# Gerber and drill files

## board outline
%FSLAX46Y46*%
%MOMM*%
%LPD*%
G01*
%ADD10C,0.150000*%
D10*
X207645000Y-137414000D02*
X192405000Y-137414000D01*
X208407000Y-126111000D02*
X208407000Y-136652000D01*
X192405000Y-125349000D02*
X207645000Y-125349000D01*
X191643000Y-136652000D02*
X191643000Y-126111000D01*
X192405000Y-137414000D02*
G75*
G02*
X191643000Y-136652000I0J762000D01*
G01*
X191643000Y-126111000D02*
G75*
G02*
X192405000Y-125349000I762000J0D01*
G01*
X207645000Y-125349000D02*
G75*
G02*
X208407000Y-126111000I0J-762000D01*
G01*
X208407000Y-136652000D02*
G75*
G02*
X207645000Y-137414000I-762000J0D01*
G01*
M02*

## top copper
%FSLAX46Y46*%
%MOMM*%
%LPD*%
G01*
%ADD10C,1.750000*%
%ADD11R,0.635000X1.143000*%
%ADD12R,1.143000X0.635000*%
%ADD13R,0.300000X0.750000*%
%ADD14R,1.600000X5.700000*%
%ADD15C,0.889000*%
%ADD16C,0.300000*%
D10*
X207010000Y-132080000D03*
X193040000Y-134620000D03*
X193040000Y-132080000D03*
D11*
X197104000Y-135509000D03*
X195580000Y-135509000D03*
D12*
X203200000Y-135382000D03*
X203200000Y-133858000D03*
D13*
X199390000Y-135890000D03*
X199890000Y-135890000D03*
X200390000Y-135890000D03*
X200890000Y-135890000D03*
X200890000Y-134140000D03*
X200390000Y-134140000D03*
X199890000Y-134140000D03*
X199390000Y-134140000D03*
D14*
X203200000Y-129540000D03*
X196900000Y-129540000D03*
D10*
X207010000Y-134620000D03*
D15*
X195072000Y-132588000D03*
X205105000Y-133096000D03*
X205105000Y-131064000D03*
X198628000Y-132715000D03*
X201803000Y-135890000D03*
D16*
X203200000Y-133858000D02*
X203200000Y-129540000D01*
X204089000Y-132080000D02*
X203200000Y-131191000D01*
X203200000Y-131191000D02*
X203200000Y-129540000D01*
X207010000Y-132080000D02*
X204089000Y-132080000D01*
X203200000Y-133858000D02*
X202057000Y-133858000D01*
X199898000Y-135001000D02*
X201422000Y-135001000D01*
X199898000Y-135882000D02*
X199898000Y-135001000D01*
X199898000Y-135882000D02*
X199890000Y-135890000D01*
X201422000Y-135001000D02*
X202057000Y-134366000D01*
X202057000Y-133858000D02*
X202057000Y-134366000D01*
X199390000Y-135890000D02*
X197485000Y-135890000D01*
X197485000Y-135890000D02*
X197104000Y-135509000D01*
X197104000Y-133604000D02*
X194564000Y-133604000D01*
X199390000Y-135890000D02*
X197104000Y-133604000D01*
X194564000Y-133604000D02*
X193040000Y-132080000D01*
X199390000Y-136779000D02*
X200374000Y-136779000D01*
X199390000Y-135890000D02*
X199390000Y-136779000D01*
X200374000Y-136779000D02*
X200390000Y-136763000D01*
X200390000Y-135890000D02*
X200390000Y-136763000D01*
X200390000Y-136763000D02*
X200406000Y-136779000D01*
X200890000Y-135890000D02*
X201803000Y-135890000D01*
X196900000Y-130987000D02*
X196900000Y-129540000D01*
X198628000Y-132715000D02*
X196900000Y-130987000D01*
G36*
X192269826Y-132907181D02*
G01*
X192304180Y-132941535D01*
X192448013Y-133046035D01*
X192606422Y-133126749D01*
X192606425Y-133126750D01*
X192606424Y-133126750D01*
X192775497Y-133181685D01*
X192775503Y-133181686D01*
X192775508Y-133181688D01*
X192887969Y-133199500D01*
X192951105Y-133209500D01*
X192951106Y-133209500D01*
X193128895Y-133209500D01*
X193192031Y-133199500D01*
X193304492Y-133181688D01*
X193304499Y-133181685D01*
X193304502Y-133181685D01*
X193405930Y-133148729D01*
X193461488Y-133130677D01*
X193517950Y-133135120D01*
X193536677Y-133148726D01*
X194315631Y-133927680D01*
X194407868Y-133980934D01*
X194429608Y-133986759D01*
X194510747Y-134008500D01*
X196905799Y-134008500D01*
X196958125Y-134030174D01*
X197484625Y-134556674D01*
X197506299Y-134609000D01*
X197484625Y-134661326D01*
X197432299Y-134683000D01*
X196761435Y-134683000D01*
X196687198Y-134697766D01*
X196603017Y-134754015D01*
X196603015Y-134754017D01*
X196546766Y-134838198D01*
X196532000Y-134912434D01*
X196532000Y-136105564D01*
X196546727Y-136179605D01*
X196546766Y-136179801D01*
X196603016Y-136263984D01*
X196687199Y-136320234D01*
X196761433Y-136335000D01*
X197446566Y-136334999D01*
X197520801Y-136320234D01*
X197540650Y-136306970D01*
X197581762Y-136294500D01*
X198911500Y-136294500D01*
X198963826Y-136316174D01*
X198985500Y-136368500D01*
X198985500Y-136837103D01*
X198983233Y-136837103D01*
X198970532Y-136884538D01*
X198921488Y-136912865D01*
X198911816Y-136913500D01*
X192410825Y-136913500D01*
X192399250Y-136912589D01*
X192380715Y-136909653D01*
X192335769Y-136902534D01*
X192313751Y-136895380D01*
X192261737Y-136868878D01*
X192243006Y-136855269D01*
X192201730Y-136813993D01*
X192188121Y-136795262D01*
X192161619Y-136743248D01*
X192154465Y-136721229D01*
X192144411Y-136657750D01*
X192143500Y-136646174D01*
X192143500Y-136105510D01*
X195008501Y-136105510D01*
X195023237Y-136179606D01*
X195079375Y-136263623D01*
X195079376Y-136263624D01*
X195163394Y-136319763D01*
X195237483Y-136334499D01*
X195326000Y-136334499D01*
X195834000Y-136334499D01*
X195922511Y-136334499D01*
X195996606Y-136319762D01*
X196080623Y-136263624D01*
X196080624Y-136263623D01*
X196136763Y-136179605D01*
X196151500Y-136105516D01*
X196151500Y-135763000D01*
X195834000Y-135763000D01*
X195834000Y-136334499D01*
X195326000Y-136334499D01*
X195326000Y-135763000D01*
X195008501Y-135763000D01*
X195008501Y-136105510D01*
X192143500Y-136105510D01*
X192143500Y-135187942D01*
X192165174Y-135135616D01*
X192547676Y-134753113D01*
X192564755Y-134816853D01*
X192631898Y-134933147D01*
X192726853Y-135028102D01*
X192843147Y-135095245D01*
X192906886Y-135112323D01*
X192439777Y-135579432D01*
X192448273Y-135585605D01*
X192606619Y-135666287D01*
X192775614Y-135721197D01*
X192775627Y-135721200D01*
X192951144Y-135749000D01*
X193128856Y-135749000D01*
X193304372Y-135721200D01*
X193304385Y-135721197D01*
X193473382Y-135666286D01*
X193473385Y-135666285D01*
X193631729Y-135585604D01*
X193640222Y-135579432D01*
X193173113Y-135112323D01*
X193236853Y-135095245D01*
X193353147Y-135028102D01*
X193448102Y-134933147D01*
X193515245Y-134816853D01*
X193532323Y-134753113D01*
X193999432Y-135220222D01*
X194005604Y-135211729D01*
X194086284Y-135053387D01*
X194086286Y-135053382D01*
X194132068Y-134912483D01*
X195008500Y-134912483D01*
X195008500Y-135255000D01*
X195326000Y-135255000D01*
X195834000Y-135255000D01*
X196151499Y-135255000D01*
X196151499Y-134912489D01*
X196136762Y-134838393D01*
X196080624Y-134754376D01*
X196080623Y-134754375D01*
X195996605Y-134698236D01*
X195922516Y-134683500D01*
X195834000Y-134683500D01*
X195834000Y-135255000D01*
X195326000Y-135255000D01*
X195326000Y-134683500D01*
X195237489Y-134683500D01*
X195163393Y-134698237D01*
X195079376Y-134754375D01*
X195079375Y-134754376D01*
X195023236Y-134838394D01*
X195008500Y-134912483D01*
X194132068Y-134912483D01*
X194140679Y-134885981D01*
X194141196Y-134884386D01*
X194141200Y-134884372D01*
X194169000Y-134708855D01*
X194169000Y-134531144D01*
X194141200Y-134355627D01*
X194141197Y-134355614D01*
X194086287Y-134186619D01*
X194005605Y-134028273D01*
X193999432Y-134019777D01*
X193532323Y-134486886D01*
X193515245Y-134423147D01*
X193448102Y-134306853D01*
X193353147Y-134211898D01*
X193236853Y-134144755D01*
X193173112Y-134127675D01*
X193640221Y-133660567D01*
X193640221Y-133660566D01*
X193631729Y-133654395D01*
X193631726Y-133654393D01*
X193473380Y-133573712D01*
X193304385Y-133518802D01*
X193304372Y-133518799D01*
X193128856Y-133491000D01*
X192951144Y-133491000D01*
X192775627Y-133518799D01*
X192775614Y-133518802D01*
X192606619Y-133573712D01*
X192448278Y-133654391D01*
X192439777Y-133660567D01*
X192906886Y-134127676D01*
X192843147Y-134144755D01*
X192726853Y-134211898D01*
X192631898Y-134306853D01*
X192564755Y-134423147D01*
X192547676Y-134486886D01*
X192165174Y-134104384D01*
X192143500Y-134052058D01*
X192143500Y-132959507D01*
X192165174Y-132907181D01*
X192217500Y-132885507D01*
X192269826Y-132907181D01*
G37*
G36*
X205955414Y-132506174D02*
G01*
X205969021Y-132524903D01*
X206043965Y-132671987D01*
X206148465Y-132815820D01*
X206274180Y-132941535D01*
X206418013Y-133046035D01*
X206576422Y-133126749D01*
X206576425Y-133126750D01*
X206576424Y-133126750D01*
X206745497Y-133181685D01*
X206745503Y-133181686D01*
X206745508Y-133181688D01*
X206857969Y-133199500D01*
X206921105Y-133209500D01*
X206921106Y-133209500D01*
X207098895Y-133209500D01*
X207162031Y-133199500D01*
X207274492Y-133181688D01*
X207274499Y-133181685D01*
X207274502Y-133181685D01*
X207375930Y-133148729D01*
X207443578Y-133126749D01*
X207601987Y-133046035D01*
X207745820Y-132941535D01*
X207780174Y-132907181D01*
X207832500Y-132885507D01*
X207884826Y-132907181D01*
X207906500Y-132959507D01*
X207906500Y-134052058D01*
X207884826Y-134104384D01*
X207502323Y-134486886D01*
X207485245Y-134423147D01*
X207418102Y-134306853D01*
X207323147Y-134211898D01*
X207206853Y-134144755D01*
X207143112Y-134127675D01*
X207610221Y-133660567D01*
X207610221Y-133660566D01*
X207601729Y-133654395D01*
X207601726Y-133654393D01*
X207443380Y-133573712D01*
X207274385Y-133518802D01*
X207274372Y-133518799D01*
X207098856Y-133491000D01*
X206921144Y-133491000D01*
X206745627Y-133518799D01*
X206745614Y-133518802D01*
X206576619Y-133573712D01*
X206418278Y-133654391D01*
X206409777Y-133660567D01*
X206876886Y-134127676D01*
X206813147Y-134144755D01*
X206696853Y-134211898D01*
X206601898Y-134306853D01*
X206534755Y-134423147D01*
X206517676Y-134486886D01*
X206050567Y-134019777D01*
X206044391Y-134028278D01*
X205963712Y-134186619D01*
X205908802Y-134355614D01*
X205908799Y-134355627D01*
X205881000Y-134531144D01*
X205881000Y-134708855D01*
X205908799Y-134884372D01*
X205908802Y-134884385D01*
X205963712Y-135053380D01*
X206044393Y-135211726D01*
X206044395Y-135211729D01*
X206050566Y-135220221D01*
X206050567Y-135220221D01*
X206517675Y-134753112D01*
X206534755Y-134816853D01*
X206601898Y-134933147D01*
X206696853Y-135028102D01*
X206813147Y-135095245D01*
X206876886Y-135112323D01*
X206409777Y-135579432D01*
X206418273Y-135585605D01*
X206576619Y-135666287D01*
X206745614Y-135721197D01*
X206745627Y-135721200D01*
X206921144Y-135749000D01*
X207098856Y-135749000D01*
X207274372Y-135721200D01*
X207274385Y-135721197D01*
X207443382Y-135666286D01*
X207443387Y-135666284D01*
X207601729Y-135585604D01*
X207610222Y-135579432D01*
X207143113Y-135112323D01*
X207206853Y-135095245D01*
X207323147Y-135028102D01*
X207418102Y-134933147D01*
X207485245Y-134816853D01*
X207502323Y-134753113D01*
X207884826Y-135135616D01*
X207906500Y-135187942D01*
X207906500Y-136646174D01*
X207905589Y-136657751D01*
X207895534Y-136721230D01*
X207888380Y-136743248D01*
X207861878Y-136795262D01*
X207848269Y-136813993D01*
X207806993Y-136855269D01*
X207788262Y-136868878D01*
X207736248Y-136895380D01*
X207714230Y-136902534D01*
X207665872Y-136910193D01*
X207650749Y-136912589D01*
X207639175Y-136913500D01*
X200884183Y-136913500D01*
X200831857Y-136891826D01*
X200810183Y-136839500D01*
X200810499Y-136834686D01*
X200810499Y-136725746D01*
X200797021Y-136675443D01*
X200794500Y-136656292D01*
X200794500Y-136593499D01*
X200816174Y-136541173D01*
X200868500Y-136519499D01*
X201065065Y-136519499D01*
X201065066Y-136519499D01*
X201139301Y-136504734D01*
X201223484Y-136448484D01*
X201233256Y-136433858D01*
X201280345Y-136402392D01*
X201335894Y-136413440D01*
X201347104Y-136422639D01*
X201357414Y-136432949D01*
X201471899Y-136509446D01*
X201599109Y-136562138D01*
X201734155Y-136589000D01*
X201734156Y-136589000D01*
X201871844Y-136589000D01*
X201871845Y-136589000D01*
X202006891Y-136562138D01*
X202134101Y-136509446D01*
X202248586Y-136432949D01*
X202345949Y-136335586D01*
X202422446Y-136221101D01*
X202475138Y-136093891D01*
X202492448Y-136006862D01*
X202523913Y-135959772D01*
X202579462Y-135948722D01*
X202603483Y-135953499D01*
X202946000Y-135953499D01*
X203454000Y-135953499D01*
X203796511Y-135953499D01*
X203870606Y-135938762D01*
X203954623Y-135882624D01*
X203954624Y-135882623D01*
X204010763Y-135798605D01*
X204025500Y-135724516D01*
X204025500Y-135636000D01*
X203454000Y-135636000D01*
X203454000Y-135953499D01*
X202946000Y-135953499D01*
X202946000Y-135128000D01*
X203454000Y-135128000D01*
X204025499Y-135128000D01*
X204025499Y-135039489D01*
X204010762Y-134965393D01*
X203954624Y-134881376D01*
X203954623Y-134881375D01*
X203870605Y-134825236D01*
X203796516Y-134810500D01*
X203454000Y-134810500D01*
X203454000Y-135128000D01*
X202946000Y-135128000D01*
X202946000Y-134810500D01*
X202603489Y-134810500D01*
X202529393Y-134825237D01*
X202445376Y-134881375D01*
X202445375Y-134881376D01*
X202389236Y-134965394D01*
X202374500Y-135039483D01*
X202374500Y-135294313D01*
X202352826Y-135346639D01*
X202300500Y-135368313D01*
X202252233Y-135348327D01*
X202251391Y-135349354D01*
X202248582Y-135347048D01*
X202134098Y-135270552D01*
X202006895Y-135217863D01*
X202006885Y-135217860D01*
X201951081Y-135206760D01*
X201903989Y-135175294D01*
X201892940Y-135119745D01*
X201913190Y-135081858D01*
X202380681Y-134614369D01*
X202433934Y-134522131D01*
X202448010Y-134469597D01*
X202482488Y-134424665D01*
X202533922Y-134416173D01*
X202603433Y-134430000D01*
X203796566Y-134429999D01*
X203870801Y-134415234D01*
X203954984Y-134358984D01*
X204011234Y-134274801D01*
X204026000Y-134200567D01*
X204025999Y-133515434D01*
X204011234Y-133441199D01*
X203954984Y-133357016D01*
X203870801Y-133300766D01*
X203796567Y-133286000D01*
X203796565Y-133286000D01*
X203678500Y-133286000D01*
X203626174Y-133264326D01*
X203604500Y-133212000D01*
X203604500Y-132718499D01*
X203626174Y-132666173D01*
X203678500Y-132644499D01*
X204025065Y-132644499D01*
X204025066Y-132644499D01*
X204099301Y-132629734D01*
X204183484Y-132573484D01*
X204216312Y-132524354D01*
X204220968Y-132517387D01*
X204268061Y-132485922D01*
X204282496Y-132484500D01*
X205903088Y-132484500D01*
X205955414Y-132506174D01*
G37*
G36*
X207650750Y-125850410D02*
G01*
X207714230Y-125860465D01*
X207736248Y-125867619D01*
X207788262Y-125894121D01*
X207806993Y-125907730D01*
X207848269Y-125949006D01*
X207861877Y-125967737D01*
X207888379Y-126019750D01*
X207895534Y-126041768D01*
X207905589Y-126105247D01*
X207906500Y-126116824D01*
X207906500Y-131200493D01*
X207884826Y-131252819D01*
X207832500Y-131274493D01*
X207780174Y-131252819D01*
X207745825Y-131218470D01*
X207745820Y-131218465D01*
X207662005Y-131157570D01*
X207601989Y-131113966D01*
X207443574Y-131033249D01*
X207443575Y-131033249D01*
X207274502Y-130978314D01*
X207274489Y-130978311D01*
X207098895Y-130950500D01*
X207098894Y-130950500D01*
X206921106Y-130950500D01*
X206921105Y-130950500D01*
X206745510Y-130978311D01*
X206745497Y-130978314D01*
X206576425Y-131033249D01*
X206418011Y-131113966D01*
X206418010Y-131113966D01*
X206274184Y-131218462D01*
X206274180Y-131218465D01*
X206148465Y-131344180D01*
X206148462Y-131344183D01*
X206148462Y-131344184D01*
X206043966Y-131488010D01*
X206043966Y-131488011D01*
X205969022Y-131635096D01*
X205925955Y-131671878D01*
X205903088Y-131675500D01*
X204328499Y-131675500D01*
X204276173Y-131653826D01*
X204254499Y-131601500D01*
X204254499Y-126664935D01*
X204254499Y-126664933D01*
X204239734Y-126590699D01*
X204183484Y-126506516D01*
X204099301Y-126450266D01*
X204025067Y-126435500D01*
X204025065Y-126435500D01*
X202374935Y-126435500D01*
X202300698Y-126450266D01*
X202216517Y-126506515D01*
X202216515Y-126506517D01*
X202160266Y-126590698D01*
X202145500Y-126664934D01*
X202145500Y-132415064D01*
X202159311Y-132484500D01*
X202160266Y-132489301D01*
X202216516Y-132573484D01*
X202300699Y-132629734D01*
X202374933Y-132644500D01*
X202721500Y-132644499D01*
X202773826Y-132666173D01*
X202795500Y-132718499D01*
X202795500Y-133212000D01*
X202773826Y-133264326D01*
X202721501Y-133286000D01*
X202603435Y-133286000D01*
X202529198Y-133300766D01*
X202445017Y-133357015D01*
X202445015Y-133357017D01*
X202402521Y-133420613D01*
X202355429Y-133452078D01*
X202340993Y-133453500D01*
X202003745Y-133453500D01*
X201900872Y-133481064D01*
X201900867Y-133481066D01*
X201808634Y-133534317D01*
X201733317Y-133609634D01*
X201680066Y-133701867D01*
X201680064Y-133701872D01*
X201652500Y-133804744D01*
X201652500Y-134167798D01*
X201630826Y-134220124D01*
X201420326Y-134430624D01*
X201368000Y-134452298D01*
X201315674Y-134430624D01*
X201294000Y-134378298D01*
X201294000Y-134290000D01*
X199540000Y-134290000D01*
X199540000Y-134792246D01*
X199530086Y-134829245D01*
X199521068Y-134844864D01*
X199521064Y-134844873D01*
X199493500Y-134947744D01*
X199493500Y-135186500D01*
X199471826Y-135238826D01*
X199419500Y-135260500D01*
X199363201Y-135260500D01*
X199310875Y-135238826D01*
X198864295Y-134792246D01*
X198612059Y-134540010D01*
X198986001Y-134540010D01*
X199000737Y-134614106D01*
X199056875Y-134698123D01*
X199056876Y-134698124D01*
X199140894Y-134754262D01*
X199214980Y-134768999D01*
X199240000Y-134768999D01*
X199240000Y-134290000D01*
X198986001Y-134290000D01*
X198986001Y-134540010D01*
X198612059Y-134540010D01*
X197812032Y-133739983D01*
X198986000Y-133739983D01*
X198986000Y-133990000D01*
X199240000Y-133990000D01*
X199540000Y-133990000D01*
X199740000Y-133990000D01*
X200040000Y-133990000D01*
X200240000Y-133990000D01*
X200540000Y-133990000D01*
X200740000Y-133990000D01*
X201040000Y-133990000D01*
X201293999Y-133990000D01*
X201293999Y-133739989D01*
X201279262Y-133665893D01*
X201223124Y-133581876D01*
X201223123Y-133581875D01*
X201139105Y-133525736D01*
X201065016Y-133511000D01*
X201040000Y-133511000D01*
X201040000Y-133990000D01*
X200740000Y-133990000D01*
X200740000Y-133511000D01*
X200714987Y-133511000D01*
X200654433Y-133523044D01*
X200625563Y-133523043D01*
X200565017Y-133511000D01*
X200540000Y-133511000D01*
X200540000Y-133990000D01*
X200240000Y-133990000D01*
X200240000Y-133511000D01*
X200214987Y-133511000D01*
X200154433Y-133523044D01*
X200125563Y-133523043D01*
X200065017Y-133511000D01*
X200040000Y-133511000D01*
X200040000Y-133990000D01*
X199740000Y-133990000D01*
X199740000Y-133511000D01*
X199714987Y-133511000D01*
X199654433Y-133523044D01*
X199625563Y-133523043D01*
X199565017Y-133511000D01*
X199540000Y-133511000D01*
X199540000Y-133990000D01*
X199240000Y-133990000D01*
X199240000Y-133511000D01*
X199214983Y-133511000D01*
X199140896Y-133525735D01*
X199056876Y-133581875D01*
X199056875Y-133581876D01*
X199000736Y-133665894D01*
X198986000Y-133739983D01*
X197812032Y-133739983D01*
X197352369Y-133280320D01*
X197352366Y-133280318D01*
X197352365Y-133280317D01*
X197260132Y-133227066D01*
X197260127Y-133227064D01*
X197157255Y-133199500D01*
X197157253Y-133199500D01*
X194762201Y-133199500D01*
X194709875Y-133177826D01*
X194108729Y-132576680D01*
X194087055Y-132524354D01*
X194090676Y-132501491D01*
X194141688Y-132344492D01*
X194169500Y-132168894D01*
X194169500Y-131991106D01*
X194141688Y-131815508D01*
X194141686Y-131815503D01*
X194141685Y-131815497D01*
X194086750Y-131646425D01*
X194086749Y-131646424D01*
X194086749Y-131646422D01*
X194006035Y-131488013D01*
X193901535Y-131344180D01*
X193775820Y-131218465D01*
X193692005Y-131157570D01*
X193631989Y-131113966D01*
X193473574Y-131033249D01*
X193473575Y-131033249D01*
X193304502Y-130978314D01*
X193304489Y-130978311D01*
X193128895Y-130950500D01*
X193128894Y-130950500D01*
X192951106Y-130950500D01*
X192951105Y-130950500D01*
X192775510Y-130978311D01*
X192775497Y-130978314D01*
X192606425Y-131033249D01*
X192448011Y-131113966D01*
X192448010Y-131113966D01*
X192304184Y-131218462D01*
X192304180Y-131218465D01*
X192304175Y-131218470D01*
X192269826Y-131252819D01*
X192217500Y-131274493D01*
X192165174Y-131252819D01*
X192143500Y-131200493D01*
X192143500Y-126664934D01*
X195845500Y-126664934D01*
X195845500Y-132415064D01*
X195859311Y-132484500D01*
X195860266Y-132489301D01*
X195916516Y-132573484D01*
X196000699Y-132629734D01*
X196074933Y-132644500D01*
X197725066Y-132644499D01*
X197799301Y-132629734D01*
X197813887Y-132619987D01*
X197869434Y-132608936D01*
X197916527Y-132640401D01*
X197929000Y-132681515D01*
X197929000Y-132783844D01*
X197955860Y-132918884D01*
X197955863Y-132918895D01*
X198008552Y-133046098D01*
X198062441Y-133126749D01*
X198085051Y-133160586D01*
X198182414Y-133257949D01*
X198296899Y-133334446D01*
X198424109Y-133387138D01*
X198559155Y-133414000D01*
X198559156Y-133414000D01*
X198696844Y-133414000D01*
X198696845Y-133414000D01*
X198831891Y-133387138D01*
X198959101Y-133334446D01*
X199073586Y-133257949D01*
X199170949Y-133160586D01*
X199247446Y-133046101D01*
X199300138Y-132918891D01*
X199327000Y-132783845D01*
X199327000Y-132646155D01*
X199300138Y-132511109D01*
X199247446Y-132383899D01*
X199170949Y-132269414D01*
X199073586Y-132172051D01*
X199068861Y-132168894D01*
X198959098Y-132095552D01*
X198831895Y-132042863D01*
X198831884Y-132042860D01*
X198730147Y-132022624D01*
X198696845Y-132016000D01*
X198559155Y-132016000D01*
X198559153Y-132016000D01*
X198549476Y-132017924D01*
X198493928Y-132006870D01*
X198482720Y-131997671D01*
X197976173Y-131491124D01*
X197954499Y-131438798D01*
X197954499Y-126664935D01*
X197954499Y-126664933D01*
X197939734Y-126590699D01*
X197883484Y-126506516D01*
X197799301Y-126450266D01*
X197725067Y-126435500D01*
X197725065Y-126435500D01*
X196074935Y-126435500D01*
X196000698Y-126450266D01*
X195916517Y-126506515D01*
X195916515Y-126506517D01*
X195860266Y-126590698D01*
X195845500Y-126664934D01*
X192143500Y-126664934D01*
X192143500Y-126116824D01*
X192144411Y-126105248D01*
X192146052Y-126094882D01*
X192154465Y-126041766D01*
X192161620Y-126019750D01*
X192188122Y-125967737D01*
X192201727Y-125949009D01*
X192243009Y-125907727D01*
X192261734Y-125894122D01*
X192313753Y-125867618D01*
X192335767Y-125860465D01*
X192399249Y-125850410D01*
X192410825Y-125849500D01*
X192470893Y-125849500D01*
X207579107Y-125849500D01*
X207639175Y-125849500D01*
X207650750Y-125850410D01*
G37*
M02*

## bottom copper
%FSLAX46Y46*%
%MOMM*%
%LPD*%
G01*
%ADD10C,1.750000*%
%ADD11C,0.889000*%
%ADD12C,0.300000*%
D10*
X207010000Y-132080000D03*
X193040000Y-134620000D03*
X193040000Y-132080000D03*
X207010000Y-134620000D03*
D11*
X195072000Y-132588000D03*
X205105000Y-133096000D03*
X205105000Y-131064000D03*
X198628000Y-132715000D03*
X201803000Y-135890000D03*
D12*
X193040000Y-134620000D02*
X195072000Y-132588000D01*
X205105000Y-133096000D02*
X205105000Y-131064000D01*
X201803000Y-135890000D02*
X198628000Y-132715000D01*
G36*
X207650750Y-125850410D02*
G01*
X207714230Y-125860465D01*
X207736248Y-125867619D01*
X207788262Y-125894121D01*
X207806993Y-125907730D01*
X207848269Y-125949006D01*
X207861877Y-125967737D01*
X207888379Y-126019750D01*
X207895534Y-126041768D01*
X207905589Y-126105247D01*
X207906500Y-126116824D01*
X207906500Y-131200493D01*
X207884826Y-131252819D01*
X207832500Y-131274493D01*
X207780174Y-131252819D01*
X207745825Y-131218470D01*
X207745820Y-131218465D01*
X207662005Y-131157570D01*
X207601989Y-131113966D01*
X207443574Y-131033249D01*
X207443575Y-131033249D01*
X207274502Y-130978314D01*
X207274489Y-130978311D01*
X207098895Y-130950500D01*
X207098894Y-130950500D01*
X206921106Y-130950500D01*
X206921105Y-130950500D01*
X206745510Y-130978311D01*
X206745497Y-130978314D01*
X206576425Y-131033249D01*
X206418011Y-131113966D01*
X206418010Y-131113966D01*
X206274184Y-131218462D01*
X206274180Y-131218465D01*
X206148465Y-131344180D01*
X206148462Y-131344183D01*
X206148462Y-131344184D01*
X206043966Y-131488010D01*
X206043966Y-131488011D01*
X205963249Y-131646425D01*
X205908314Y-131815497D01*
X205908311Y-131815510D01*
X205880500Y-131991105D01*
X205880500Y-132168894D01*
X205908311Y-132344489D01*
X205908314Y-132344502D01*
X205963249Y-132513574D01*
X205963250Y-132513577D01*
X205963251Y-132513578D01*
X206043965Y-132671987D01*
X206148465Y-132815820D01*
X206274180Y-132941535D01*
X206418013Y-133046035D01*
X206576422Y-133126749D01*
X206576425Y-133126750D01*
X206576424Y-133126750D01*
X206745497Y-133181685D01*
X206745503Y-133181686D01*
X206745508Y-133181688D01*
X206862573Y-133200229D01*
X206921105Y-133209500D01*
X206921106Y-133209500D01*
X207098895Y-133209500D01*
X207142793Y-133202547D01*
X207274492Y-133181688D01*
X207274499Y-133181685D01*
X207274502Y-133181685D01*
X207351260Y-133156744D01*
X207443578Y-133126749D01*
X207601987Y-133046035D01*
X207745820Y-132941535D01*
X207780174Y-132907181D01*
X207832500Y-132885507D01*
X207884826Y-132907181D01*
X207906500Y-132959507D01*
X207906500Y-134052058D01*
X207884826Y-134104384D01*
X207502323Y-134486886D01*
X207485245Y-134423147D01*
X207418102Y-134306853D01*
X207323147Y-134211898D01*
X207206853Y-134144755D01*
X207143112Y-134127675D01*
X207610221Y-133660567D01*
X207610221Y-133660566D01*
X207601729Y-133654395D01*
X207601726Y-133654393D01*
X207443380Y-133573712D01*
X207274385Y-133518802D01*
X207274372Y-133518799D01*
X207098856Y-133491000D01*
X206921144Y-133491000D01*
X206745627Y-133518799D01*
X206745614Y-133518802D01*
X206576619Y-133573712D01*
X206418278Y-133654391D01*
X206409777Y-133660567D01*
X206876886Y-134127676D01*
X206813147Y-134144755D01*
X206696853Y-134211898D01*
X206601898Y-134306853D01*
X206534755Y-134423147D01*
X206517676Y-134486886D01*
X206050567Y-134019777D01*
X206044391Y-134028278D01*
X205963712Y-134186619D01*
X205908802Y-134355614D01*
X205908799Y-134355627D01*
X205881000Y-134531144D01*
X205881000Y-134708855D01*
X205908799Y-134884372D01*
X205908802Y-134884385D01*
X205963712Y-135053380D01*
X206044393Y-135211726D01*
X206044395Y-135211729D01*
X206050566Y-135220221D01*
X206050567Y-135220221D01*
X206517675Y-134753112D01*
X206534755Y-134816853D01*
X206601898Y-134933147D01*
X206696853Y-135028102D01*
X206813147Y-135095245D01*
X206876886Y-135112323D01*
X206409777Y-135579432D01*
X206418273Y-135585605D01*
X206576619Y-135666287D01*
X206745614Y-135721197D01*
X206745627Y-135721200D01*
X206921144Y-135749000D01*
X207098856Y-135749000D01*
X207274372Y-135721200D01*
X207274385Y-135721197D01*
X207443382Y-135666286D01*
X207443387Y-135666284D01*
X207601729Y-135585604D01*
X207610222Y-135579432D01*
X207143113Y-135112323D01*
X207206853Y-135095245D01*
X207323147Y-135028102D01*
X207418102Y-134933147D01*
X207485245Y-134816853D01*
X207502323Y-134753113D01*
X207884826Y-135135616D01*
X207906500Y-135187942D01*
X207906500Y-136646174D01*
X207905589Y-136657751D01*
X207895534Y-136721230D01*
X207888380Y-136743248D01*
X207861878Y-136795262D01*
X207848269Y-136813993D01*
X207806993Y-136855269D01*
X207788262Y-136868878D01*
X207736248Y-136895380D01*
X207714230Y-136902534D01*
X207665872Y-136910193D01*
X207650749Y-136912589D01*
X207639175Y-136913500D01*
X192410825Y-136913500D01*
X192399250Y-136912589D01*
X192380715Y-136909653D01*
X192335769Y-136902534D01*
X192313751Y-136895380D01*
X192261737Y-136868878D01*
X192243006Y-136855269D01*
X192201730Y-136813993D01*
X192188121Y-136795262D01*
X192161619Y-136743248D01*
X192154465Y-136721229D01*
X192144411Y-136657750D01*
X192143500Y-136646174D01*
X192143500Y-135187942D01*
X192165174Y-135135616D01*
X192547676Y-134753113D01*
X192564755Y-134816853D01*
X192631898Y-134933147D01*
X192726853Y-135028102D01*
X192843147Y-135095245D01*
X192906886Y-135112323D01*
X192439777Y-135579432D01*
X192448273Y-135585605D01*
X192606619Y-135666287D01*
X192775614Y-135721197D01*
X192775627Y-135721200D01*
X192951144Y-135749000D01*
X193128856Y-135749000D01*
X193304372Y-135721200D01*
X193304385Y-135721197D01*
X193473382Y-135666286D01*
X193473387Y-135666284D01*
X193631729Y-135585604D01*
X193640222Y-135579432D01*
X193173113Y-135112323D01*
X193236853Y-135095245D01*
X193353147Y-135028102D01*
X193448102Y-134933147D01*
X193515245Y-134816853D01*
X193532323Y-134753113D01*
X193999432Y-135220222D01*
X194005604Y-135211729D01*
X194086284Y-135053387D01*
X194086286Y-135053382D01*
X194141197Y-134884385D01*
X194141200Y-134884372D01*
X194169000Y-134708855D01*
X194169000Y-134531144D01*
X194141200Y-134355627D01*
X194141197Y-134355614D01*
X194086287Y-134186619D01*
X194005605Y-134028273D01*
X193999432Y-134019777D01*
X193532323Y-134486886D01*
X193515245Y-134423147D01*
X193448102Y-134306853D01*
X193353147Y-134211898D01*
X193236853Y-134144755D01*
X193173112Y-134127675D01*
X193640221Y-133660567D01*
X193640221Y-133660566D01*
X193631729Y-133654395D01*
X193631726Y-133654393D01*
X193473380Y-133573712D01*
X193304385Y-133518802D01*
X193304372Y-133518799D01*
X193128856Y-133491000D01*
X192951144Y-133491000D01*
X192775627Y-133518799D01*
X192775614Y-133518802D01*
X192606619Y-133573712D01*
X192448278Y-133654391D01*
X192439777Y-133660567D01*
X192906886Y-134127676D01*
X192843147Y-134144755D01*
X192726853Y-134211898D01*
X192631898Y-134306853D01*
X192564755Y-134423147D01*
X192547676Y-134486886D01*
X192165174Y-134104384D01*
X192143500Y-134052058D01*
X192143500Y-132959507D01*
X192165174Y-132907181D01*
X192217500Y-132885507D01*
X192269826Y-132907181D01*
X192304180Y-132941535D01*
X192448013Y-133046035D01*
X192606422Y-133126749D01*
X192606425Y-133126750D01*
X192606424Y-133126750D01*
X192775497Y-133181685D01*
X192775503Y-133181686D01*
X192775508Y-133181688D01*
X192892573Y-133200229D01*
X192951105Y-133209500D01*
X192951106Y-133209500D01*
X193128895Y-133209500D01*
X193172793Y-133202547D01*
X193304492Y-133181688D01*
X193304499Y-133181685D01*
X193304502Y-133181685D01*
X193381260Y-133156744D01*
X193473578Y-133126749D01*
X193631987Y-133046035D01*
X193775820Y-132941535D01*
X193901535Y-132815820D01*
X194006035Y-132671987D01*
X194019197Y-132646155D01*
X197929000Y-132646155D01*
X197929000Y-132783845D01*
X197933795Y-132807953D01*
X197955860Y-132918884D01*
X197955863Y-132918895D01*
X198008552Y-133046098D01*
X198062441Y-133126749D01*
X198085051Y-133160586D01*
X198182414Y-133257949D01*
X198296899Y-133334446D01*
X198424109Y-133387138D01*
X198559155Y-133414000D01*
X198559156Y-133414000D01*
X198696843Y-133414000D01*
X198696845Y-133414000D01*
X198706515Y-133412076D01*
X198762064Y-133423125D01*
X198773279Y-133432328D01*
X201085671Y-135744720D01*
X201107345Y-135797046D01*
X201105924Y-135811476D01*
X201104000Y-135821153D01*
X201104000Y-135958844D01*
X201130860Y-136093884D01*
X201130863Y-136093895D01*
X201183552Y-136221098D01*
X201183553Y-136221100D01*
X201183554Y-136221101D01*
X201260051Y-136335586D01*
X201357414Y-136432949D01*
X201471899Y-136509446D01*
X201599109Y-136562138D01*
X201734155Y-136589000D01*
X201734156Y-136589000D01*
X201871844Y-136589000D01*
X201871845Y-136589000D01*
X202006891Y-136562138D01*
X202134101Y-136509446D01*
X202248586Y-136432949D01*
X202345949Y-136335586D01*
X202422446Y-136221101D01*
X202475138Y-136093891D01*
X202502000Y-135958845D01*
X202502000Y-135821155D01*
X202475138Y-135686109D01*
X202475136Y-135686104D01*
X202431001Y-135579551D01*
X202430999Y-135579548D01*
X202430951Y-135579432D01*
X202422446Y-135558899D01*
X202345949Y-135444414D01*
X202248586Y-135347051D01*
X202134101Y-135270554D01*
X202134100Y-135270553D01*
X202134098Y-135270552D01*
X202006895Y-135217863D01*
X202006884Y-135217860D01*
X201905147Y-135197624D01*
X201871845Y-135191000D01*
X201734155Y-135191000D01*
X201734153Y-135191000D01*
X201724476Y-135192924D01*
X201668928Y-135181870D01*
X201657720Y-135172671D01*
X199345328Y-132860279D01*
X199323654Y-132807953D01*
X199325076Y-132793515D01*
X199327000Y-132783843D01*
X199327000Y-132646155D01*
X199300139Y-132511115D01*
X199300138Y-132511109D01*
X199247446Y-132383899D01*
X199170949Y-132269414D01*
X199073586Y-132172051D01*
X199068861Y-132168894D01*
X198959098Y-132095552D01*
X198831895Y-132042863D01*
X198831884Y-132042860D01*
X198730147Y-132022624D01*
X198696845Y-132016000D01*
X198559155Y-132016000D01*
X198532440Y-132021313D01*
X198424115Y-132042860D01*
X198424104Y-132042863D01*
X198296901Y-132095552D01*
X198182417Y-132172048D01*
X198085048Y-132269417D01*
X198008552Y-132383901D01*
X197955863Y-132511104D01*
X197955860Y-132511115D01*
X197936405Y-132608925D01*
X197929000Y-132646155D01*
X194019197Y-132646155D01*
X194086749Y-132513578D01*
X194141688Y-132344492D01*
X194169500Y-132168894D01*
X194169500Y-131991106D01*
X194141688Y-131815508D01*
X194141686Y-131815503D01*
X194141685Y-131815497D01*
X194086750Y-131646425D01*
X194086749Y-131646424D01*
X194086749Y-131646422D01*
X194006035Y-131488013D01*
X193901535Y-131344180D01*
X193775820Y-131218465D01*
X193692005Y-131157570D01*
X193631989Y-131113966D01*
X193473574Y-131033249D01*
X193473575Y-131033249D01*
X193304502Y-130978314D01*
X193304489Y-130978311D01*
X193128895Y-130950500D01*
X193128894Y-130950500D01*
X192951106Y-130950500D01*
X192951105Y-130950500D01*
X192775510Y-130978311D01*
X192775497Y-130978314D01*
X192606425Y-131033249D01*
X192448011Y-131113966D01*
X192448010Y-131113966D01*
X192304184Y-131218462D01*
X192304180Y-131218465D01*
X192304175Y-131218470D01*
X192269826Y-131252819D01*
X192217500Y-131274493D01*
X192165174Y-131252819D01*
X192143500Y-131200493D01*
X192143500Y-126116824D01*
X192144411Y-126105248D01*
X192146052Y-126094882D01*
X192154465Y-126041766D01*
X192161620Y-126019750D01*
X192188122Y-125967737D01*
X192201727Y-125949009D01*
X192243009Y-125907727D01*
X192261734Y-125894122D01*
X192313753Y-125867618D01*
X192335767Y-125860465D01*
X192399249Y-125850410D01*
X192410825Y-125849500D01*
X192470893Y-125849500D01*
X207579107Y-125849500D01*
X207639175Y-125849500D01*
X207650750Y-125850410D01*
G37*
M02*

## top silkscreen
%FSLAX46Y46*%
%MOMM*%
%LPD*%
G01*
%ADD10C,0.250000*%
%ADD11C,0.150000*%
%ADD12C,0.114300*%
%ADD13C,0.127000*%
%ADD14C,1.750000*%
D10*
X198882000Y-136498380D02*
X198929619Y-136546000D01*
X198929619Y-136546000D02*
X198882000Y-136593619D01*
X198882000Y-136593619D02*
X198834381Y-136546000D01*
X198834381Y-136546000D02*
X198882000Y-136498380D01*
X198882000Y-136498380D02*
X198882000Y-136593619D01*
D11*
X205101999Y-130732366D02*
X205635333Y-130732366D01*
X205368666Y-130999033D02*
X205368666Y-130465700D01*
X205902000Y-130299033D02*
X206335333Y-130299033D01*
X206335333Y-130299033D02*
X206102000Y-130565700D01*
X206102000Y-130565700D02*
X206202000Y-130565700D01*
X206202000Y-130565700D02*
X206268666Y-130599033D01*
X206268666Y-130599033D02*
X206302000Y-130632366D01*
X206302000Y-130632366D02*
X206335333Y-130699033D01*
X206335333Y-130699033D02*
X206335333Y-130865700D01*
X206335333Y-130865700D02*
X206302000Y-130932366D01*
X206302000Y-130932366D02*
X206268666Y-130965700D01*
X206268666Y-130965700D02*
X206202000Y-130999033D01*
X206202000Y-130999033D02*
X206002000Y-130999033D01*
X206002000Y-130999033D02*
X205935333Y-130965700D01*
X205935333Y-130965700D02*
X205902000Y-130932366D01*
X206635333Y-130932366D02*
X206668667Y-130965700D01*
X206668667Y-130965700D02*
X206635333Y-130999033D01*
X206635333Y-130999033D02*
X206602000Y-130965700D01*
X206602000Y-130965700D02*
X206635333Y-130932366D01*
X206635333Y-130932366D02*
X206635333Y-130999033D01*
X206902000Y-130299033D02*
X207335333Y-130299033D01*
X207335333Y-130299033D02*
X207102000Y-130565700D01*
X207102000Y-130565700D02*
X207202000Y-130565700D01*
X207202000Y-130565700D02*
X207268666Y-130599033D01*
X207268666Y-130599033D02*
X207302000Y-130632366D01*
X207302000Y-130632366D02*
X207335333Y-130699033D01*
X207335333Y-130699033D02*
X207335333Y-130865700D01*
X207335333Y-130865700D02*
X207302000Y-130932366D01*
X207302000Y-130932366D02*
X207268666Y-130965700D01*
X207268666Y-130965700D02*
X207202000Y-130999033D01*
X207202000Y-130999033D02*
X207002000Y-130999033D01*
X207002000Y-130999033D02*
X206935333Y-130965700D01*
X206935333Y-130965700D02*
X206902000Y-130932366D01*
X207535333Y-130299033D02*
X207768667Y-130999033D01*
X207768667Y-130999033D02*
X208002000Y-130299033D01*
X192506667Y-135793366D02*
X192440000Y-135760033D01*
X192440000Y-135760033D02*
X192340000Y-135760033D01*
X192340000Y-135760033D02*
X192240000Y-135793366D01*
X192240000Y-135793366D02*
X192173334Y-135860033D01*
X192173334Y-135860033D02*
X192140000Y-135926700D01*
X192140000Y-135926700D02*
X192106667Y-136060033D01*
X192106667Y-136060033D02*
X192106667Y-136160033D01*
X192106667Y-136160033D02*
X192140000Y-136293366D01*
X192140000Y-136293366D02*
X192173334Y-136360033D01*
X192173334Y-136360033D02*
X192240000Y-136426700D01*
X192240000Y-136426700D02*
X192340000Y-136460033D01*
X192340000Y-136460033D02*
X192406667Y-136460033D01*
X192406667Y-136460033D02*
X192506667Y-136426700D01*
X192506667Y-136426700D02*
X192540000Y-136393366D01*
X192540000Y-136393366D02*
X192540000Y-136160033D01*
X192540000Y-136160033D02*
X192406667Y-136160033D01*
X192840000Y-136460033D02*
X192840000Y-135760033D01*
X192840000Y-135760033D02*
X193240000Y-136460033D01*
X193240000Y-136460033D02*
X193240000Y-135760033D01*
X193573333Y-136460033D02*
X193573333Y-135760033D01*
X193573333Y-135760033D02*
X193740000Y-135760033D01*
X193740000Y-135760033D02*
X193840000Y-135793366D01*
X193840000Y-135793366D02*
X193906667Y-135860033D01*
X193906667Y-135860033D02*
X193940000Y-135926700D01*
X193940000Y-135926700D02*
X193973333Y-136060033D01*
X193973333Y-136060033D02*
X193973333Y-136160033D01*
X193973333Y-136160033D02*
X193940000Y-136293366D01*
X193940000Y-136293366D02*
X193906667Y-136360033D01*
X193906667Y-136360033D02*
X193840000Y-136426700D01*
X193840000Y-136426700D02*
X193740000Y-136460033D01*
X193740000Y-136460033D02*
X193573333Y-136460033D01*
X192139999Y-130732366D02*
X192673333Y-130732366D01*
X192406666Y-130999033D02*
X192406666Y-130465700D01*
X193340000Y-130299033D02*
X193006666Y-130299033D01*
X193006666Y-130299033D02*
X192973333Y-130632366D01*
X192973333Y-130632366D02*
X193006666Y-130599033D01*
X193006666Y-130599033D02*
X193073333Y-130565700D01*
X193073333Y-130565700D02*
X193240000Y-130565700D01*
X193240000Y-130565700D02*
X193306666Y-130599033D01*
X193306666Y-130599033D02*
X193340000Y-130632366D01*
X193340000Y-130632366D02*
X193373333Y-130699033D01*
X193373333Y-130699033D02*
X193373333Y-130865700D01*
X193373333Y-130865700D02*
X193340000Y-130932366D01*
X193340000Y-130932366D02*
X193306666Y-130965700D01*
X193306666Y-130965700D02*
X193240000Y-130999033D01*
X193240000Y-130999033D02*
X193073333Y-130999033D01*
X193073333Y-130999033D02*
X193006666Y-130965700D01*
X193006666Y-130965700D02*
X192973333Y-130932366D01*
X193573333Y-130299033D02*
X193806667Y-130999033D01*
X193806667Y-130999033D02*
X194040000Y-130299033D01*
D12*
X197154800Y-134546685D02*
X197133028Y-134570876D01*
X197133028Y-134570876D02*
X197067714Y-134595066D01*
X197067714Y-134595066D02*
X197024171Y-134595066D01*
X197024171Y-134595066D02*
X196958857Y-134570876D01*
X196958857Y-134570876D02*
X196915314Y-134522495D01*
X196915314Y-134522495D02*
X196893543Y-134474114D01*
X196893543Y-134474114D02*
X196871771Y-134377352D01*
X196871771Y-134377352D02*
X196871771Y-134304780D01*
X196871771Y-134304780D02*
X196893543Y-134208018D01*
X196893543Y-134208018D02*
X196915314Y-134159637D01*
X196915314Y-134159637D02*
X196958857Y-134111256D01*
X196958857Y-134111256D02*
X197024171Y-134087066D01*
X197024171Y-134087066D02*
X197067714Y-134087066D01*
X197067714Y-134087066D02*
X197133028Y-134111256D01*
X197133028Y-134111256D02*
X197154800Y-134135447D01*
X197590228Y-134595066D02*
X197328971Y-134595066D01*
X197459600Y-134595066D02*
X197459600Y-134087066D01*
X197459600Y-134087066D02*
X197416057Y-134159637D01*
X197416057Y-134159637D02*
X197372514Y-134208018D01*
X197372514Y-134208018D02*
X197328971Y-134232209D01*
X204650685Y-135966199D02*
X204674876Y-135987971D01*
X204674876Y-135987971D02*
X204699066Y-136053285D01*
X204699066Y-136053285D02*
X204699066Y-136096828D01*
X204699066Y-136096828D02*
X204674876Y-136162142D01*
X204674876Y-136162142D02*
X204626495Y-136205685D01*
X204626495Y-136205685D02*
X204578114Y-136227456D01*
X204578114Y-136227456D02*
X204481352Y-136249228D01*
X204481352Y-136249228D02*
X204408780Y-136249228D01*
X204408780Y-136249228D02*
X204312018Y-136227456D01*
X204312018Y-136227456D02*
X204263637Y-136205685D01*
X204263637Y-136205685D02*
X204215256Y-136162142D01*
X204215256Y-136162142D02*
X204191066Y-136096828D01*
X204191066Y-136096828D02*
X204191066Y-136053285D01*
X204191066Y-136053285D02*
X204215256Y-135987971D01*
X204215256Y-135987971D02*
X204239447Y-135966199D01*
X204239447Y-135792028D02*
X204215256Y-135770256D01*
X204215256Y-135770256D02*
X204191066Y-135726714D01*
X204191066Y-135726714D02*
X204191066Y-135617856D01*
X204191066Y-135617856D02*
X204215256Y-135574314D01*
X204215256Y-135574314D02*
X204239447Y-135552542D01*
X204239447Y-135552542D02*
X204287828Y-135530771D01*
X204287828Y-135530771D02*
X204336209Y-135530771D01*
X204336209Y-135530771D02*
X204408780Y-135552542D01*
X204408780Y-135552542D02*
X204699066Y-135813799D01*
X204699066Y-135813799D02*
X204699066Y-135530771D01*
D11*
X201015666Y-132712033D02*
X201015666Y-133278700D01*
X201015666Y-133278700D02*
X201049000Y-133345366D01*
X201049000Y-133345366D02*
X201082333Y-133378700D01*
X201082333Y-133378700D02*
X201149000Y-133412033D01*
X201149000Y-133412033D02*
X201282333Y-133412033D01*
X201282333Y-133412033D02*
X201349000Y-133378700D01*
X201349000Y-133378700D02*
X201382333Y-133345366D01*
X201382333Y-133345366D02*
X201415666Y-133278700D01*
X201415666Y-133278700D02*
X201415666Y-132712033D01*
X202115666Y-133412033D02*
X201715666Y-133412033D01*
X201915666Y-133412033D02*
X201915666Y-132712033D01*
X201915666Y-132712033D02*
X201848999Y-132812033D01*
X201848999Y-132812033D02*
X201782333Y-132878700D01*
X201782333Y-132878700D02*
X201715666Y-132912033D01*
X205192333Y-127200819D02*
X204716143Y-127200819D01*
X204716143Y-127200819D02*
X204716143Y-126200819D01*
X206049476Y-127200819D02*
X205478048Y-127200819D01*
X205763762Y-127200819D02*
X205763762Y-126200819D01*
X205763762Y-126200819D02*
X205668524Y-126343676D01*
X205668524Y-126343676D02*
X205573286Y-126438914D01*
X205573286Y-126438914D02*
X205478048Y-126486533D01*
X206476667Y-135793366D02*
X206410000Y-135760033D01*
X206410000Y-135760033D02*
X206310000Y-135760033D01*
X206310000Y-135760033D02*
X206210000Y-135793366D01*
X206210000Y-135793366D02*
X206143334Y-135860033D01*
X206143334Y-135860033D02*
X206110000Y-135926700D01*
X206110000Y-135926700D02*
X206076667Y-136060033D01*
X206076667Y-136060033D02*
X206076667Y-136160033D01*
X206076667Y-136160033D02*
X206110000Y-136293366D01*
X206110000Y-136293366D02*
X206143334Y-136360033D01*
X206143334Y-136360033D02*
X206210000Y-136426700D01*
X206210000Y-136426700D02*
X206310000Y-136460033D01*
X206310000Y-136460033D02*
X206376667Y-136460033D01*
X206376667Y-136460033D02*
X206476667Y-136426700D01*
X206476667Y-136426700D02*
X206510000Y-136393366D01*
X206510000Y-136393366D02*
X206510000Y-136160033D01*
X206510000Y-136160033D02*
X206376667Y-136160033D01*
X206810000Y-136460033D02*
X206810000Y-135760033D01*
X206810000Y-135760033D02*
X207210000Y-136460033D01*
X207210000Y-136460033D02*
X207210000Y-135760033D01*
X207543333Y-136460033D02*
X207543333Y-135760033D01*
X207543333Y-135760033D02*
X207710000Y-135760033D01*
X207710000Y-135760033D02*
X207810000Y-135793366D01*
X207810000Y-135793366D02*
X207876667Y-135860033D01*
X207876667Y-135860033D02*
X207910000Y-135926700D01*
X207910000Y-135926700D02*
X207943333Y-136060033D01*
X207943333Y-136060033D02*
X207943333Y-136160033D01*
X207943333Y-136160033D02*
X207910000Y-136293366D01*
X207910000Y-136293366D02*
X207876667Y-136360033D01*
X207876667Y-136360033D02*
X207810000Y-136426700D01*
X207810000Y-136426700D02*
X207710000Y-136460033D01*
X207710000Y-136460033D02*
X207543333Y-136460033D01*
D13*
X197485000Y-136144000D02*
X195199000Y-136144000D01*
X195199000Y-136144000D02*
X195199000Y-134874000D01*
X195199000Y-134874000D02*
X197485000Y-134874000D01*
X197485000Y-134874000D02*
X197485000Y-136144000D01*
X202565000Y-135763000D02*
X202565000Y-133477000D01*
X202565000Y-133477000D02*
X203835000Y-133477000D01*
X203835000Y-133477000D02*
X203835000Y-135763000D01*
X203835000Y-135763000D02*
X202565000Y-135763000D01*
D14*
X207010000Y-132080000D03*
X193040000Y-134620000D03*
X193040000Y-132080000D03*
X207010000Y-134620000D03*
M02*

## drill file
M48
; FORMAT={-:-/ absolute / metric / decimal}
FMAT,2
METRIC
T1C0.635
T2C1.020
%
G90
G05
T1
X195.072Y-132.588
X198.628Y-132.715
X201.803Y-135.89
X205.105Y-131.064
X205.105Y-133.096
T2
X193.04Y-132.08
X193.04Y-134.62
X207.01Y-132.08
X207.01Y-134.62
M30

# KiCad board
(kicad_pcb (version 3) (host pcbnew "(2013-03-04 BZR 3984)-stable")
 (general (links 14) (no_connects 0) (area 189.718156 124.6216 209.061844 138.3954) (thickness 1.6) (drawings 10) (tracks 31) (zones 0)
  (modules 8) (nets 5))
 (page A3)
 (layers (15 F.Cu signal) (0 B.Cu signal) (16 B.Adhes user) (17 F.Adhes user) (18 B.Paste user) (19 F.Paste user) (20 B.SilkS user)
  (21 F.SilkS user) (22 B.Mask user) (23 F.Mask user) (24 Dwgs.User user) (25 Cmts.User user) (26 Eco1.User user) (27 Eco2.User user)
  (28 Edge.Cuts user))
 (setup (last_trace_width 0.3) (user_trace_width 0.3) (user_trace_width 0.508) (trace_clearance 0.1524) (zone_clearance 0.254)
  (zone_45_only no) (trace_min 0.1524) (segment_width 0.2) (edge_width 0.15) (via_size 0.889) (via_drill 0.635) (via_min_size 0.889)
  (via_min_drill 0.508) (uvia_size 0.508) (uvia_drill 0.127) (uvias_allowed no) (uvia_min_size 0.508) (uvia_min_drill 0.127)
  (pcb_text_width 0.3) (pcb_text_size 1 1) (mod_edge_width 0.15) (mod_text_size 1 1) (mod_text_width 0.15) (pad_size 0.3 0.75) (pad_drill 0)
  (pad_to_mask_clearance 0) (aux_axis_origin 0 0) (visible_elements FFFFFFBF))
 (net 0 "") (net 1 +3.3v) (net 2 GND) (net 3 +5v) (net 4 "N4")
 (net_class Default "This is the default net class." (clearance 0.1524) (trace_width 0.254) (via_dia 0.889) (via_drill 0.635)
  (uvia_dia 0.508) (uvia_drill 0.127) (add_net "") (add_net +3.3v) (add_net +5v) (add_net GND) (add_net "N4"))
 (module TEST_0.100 (layer F.Cu) (at 207.01 132.08)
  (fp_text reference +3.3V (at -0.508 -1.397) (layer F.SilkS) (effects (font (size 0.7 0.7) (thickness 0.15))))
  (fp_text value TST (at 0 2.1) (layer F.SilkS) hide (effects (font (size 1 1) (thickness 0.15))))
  (pad 1 thru_hole circle (at 0 0) (size 1.75 1.75) (drill 1.02) (layers *.Cu *.Mask F.SilkS) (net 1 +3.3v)))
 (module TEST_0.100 (layer F.Cu) (at 193.04 134.62)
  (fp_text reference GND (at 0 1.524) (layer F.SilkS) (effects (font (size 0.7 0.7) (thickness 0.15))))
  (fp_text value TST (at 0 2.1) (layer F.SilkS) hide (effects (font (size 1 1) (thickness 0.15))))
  (pad 1 thru_hole circle (at 0 0) (size 1.75 1.75) (drill 1.02) (layers *.Cu *.Mask F.SilkS) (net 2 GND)))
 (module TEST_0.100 (layer F.Cu) (at 193.04 132.08)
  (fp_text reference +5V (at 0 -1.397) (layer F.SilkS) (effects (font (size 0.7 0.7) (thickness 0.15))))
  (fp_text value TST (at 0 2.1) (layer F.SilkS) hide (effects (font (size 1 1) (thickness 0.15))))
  (pad 1 thru_hole circle (at 0 0) (size 1.75 1.75) (drill 1.02) (layers *.Cu *.Mask F.SilkS) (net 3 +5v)))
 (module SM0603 (layer F.Cu) (at 196.342 135.509 180)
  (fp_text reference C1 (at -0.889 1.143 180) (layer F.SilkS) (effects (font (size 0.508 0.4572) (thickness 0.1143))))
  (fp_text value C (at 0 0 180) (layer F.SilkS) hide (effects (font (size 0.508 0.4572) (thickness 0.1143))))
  (fp_line (start -1.143 -0.635) (end 1.143 -0.635) (layer F.SilkS) (width 0.127))
  (fp_line (start 1.143 -0.635) (end 1.143 0.635) (layer F.SilkS) (width 0.127))
  (fp_line (start 1.143 0.635) (end -1.143 0.635) (layer F.SilkS) (width 0.127))
  (fp_line (start -1.143 0.635) (end -1.143 -0.635) (layer F.SilkS) (width 0.127))
  (pad 1 smd rect (at -0.762 0 180) (size 0.635 1.143) (layers F.Cu F.Paste F.Mask) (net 3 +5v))
  (pad 2 smd rect (at 0.762 0 180) (size 0.635 1.143) (layers F.Cu F.Paste F.Mask) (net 2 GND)))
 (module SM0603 (layer F.Cu) (at 203.2 134.62 90)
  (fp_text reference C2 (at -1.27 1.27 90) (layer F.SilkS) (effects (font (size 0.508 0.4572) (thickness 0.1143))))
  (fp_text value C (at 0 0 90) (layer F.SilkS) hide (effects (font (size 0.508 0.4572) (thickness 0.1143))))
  (fp_line (start -1.143 -0.635) (end 1.143 -0.635) (layer F.SilkS) (width 0.127))
  (fp_line (start 1.143 -0.635) (end 1.143 0.635) (layer F.SilkS) (width 0.127))
  (fp_line (start 1.143 0.635) (end -1.143 0.635) (layer F.SilkS) (width 0.127))
  (fp_line (start -1.143 0.635) (end -1.143 -0.635) (layer F.SilkS) (width 0.127))
  (pad 1 smd rect (at -0.762 0 90) (size 0.635 1.143) (layers F.Cu F.Paste F.Mask) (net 2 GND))
  (pad 2 smd rect (at 0.762 0 90) (size 0.635 1.143) (layers F.Cu F.Paste F.Mask) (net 1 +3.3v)))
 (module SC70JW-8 (layer F.Cu) (at 199.39 135.89)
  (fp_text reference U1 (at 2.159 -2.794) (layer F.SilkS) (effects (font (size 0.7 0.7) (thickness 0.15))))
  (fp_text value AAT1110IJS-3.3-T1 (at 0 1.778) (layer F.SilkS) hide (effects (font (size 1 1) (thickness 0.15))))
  (pad 1 smd rect (at 0 0) (size 0.3 0.75) (layers F.Cu F.Paste F.Mask) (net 3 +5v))
  (pad 2 smd rect (at 0.5 0) (size 0.3 0.75) (layers F.Cu F.Paste F.Mask) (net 1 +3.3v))
  (pad 3 smd rect (at 1 0) (size 0.3 0.75) (layers F.Cu F.Paste F.Mask) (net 3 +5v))
  (pad 4 smd rect (at 1.5 0) (size 0.3 0.75) (layers F.Cu F.Paste F.Mask) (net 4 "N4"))
  (pad 5 smd rect (at 1.5 -1.75) (size 0.3 0.75) (layers F.Cu F.Paste F.Mask) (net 2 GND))
  (pad 6 smd rect (at 1 -1.75) (size 0.3 0.75) (layers F.Cu F.Paste F.Mask) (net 2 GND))
  (pad 7 smd rect (at 0.5 -1.75) (size 0.3 0.75) (layers F.Cu F.Paste F.Mask) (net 2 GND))
  (pad 8 smd rect (at 0 -1.75) (size 0.3 0.75) (layers F.Cu F.Paste F.Mask) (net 2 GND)))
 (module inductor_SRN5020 (layer F.Cu) (at 203.2 129.54 180)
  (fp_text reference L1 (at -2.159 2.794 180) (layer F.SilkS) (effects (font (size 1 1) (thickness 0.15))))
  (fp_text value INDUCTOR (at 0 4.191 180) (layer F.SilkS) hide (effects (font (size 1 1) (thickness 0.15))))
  (pad 1 smd rect (at 0 0 180) (size 1.6 5.7) (layers F.Cu F.Paste F.Mask) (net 1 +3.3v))
  (pad 2 smd rect (at 6.3 0 180) (size 1.6 5.7) (layers F.Cu F.Paste F.Mask) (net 4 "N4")))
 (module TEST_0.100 (layer F.Cu) (at 207.01 134.62)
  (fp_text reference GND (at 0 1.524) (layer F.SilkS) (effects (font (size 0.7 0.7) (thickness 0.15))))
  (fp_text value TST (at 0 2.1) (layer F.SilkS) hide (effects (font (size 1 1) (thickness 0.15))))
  (pad 1 thru_hole circle (at 0 0) (size 1.75 1.75) (drill 1.02) (layers *.Cu *.Mask F.SilkS) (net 2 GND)))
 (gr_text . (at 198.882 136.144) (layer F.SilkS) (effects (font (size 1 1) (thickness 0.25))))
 (gr_line (start 207.645 137.414) (end 192.405 137.414) (angle 90) (layer Edge.Cuts) (width 0.15))
 (gr_line (start 208.407 126.111) (end 208.407 136.652) (angle 90) (layer Edge.Cuts) (width 0.15))
 (gr_line (start 192.405 125.349) (end 207.645 125.349) (angle 90) (layer Edge.Cuts) (width 0.15))
 (gr_line (start 191.643 136.652) (end 191.643 126.111) (angle 90) (layer Edge.Cuts) (width 0.15))
 (gr_arc (start 192.405 136.652) (end 192.405 137.414) (angle 90) (layer Edge.Cuts) (width 0.15))
 (gr_arc (start 192.405 126.111) (end 191.643 126.111) (angle 90) (layer Edge.Cuts) (width 0.15))
 (gr_arc (start 207.645 126.111) (end 207.645 125.349) (angle 90) (layer Edge.Cuts) (width 0.15))
 (gr_arc (start 207.645 136.652) (end 208.407 136.652) (angle 90) (layer Edge.Cuts) (width 0.15))
 (segment (start 203.2 133.858) (end 203.2 129.54) (width 0.3) (layer F.Cu) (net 1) (status C00000))
 (segment (start 204.089 132.08) (end 203.2 131.191) (width 0.3) (layer F.Cu) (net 1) (status 800000))
 (segment (start 203.2 131.191) (end 203.2 129.54) (width 0.3) (layer F.Cu) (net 1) (status C00000))
 (segment (start 207.01 132.08) (end 204.089 132.08) (width 0.3) (layer F.Cu) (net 1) (status 400000))
 (segment (start 203.2 133.858) (end 202.057 133.858) (width 0.3) (layer F.Cu) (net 1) (status 400000))
 (segment (start 199.898 135.001) (end 201.422 135.001) (width 0.3) (layer F.Cu) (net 1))
 (segment (start 199.898 135.882) (end 199.898 135.001) (width 0.3) (layer F.Cu) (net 1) (status 400000))
 (segment (start 199.898 135.882) (end 199.89 135.89) (width 0.3) (layer F.Cu) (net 1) (status C00000))
 (segment (start 201.422 135.001) (end 202.057 134.366) (width 0.3) (layer F.Cu) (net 1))
 (segment (start 202.057 133.858) (end 202.057 134.366) (width 0.3) (layer F.Cu) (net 1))
 (segment (start 199.39 135.89) (end 197.485 135.89) (width 0.3) (layer F.Cu) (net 3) (status 400000))
 (segment (start 197.485 135.89) (end 197.104 135.509) (width 0.3) (layer F.Cu) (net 3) (status 800000))
 (segment (start 197.104 133.604) (end 194.564 133.604) (width 0.3) (layer F.Cu) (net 3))
 (segment (start 199.39 135.89) (end 197.104 133.604) (width 0.3) (layer F.Cu) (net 3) (status 400000))
 (segment (start 194.564 133.604) (end 193.04 132.08) (width 0.3) (layer F.Cu) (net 3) (status 800000))
 (segment (start 199.39 136.779) (end 200.374 136.779) (width 0.3) (layer F.Cu) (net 3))
 (segment (start 199.39 135.89) (end 199.39 136.779) (width 0.3) (layer F.Cu) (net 3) (status 400000))
 (segment (start 200.374 136.779) (end 200.39 136.763) (width 0.3) (layer F.Cu) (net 3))
 (segment (start 200.39 135.89) (end 200.39 136.763) (width 0.3) (layer F.Cu) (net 3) (status 400000))
 (segment (start 200.39 136.763) (end 200.406 136.779) (width 0.3) (layer F.Cu) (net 3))
 (segment (start 193.04 134.62) (end 195.072 132.588) (width 0.3) (layer B.Cu) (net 2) (status 400000))
 (via (at 195.072 132.588) (size 0.889) (layers F.Cu B.Cu) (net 2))
 (via (at 205.105 133.096) (size 0.889) (layers F.Cu B.Cu) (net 2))
 (via (at 205.105 131.064) (size 0.889) (layers F.Cu B.Cu) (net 2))
 (segment (start 205.105 133.096) (end 205.105 131.064) (width 0.3) (layer B.Cu) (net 2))
 (segment (start 200.89 135.89) (end 201.803 135.89) (width 0.3) (layer F.Cu) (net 4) (status 400000))
 (segment (start 196.9 130.987) (end 196.9 129.54) (width 0.3) (layer F.Cu) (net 4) (status C00000))
 (segment (start 198.628 132.715) (end 196.9 130.987) (width 0.3) (layer F.Cu) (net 4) (status 800000))
 (via (at 198.628 132.715) (size 0.889) (layers F.Cu B.Cu) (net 4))
 (segment (start 201.803 135.89) (end 198.628 132.715) (width 0.3) (layer B.Cu) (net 4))
 (via (at 201.803 135.89) (size 0.889) (layers F.Cu B.Cu) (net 4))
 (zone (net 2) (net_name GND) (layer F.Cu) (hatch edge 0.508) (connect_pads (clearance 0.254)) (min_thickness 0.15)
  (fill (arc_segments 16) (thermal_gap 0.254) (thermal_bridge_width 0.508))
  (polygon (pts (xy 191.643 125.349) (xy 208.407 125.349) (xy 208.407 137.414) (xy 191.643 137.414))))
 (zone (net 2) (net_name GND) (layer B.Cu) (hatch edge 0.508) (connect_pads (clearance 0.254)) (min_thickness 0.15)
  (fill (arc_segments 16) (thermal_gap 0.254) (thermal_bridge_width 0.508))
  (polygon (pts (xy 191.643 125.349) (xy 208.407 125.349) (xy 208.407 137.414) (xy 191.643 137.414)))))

